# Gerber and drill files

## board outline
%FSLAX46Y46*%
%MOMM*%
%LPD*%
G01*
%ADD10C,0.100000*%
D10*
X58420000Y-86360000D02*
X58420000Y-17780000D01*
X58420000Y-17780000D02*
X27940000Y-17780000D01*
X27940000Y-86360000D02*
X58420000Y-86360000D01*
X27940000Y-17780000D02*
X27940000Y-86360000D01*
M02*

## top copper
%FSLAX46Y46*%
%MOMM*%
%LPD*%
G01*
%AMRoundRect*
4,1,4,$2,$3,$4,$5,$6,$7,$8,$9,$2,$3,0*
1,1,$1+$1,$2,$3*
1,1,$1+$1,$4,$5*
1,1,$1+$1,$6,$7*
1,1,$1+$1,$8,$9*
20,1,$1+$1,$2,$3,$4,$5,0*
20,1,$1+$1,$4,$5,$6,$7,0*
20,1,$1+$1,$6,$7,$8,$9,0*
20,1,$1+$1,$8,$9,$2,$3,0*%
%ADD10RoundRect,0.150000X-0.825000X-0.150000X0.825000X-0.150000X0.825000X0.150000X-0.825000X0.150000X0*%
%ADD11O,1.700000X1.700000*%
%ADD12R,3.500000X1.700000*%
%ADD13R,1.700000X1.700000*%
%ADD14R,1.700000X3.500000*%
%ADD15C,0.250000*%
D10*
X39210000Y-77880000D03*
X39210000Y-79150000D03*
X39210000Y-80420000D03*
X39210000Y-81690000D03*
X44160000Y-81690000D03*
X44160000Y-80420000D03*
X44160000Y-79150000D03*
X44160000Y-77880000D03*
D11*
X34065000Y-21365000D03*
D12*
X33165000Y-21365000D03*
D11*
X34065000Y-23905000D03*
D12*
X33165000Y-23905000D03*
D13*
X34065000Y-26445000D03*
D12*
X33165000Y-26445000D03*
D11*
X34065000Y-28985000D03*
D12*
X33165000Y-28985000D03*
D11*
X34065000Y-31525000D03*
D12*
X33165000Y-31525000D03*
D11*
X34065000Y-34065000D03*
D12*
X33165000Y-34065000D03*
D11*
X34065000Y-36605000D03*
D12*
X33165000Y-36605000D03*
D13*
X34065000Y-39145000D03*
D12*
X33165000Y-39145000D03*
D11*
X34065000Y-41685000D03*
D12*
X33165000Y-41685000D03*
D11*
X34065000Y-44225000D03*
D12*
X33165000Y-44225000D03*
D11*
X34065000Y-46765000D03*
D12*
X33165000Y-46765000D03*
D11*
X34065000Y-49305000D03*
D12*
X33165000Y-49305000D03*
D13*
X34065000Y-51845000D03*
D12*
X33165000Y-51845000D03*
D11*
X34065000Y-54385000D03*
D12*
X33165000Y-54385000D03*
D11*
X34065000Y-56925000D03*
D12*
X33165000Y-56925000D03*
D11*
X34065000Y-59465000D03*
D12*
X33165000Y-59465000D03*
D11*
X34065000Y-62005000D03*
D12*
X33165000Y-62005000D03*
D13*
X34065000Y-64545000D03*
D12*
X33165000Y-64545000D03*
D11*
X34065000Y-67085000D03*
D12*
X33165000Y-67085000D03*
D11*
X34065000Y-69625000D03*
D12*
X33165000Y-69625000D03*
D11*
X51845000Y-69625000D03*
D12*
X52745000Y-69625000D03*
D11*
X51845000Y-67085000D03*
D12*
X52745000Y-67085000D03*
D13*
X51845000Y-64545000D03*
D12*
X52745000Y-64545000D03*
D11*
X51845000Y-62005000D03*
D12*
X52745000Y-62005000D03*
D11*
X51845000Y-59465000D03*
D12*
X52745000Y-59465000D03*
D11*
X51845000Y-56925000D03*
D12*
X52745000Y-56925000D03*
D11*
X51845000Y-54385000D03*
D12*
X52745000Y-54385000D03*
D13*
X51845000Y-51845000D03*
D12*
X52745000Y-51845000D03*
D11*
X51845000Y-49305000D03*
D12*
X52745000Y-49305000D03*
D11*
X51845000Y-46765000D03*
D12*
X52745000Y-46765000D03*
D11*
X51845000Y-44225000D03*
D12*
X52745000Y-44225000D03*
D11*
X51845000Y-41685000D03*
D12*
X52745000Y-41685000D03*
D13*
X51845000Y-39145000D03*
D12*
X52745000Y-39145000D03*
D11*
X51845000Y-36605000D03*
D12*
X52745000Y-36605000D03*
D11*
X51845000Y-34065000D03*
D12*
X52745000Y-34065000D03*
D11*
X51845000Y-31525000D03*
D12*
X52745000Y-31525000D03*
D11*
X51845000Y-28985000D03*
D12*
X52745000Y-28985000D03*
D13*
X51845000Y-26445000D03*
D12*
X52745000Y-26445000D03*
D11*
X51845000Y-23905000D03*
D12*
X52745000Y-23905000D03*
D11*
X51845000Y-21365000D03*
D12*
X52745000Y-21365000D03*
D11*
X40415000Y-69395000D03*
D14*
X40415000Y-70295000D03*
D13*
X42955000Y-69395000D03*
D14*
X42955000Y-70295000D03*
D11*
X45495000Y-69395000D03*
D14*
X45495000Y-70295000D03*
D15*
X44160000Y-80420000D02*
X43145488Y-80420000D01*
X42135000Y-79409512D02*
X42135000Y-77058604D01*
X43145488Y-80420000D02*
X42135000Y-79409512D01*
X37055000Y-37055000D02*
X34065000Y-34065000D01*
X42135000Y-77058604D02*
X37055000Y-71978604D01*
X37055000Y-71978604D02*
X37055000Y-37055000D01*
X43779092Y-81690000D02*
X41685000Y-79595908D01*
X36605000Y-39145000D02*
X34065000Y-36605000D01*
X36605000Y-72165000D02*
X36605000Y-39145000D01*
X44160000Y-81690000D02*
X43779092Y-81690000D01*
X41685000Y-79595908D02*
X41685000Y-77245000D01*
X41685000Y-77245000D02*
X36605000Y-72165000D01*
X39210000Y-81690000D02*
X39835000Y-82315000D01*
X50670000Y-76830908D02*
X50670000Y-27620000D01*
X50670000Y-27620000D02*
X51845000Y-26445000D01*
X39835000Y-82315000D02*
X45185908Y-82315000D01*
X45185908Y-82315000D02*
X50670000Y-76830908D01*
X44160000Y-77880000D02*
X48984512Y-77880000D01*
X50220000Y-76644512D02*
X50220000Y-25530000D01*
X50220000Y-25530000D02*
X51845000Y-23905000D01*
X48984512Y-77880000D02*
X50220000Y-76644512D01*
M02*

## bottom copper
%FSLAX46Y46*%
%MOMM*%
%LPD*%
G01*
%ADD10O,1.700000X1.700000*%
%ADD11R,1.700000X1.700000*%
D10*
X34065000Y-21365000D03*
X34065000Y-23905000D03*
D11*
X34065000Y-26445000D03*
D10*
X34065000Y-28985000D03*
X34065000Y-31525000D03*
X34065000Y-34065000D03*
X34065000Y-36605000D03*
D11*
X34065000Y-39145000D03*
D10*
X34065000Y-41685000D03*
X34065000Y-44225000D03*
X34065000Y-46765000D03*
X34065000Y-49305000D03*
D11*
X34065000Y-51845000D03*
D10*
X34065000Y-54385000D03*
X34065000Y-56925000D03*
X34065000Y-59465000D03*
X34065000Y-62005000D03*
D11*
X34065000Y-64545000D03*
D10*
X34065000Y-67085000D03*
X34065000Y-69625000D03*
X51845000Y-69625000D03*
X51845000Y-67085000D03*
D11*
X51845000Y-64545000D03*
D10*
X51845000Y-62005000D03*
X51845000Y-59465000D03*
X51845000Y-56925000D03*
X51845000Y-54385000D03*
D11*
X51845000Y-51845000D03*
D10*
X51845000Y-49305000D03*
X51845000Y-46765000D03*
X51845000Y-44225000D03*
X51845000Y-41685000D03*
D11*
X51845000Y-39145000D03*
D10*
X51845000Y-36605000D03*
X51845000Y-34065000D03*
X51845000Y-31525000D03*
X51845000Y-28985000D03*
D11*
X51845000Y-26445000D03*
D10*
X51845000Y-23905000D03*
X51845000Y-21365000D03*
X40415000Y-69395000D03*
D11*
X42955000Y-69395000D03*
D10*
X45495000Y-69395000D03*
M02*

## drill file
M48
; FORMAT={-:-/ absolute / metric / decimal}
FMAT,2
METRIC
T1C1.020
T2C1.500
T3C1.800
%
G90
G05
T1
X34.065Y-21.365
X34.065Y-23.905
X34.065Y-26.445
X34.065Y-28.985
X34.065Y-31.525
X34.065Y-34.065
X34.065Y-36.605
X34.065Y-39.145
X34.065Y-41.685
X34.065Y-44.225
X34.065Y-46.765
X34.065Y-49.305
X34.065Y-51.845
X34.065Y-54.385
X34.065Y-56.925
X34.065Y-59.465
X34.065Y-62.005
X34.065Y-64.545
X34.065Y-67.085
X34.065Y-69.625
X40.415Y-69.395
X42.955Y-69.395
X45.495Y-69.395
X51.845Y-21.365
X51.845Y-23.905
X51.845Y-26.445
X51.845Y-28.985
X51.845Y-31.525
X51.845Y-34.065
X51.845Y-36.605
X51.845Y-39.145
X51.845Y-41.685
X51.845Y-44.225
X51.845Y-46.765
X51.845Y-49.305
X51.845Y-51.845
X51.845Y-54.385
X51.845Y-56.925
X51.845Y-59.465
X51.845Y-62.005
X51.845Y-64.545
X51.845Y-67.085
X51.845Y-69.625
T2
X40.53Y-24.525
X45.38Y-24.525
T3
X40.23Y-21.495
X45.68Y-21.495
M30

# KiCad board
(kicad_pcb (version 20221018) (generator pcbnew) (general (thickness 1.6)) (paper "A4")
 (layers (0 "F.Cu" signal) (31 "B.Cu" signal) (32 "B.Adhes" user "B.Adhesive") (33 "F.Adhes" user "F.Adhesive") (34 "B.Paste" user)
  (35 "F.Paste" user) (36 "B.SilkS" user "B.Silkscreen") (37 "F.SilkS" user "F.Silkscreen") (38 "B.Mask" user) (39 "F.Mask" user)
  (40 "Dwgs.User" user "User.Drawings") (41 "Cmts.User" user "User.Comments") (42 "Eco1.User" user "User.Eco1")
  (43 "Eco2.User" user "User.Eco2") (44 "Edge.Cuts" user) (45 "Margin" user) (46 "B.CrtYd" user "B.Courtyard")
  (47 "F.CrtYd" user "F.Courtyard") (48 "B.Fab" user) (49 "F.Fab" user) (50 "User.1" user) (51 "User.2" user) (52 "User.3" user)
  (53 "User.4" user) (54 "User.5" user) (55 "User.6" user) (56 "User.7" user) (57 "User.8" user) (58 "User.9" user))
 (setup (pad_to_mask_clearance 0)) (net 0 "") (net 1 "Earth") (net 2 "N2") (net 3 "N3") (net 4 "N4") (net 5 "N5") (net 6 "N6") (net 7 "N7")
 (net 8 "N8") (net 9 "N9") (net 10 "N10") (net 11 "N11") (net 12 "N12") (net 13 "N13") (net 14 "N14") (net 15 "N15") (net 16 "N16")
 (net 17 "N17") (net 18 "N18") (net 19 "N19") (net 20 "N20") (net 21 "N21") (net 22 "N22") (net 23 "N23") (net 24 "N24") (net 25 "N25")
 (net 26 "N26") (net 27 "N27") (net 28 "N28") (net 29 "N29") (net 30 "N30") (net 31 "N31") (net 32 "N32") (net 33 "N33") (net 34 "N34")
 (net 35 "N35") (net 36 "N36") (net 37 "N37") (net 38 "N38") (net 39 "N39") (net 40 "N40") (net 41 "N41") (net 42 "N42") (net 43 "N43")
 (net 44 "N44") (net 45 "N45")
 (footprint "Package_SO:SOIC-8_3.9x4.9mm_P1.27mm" (layer "F.Cu") (at 41.685 79.785)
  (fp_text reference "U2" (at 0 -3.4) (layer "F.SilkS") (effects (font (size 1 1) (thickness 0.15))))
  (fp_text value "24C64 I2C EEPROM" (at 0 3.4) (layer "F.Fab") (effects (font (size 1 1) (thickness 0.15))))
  (pad "1" smd roundrect (at -2.475 -1.905) (size 1.95 0.6) (layers "F.Cu" "F.Paste" "F.Mask") (roundrect_rratio 0.25) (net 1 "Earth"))
  (pad "2" smd roundrect (at -2.475 -0.635) (size 1.95 0.6) (layers "F.Cu" "F.Paste" "F.Mask") (roundrect_rratio 0.25) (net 1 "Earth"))
  (pad "3" smd roundrect (at -2.475 0.635) (size 1.95 0.6) (layers "F.Cu" "F.Paste" "F.Mask") (roundrect_rratio 0.25) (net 1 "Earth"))
  (pad "4" smd roundrect (at -2.475 1.905) (size 1.95 0.6) (layers "F.Cu" "F.Paste" "F.Mask") (roundrect_rratio 0.25) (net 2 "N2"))
  (pad "5" smd roundrect (at 2.475 1.905) (size 1.95 0.6) (layers "F.Cu" "F.Paste" "F.Mask") (roundrect_rratio 0.25) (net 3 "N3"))
  (pad "6" smd roundrect (at 2.475 0.635) (size 1.95 0.6) (layers "F.Cu" "F.Paste" "F.Mask") (roundrect_rratio 0.25) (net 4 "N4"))
  (pad "7" smd roundrect (at 2.475 -0.635) (size 1.95 0.6) (layers "F.Cu" "F.Paste" "F.Mask") (roundrect_rratio 0.25) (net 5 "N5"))
  (pad "8" smd roundrect (at 2.475 -1.905) (size 1.95 0.6) (layers "F.Cu" "F.Paste" "F.Mask") (roundrect_rratio 0.25) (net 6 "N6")))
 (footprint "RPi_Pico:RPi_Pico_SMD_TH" (layer "F.Cu") (at 42.955 45.495)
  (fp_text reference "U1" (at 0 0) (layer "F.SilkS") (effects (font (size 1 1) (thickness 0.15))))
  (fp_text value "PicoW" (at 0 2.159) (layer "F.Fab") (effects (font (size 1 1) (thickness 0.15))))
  (pad "" np_thru_hole oval (at -2.725 -24) (size 1.8 1.8) (drill 1.8) (layers "*.Cu" "*.Mask"))
  (pad "" np_thru_hole oval (at -2.425 -20.97) (size 1.5 1.5) (drill 1.5) (layers "*.Cu" "*.Mask"))
  (pad "" np_thru_hole oval (at 2.425 -20.97) (size 1.5 1.5) (drill 1.5) (layers "*.Cu" "*.Mask"))
  (pad "" np_thru_hole oval (at 2.725 -24) (size 1.8 1.8) (drill 1.8) (layers "*.Cu" "*.Mask"))
  (pad "1" thru_hole oval (at -8.89 -24.13) (size 1.7 1.7) (drill 1.02) (layers "*.Cu" "*.Mask") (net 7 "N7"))
  (pad "1" smd rect (at -8.89 -24.13) (size 3.5 1.7) (drill (offset -0.9 0)) (layers "F.Cu" "F.Mask") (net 7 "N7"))
  (pad "2" thru_hole oval (at -8.89 -21.59) (size 1.7 1.7) (drill 1.02) (layers "*.Cu" "*.Mask") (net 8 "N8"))
  (pad "2" smd rect (at -8.89 -21.59) (size 3.5 1.7) (drill (offset -0.9 0)) (layers "F.Cu" "F.Mask") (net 8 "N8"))
  (pad "3" thru_hole rect (at -8.89 -19.05) (size 1.7 1.7) (drill 1.02) (layers "*.Cu" "*.Mask") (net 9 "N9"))
  (pad "3" smd rect (at -8.89 -19.05) (size 3.5 1.7) (drill (offset -0.9 0)) (layers "F.Cu" "F.Mask") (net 9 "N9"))
  (pad "4" thru_hole oval (at -8.89 -16.51) (size 1.7 1.7) (drill 1.02) (layers "*.Cu" "*.Mask") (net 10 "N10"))
  (pad "4" smd rect (at -8.89 -16.51) (size 3.5 1.7) (drill (offset -0.9 0)) (layers "F.Cu" "F.Mask") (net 10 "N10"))
  (pad "5" thru_hole oval (at -8.89 -13.97) (size 1.7 1.7) (drill 1.02) (layers "*.Cu" "*.Mask") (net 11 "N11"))
  (pad "5" smd rect (at -8.89 -13.97) (size 3.5 1.7) (drill (offset -0.9 0)) (layers "F.Cu" "F.Mask") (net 11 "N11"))
  (pad "6" thru_hole oval (at -8.89 -11.43) (size 1.7 1.7) (drill 1.02) (layers "*.Cu" "*.Mask") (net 4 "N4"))
  (pad "6" smd rect (at -8.89 -11.43) (size 3.5 1.7) (drill (offset -0.9 0)) (layers "F.Cu" "F.Mask") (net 4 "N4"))
  (pad "7" thru_hole oval (at -8.89 -8.89) (size 1.7 1.7) (drill 1.02) (layers "*.Cu" "*.Mask") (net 3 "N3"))
  (pad "7" smd rect (at -8.89 -8.89) (size 3.5 1.7) (drill (offset -0.9 0)) (layers "F.Cu" "F.Mask") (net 3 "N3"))
  (pad "8" thru_hole rect (at -8.89 -6.35) (size 1.7 1.7) (drill 1.02) (layers "*.Cu" "*.Mask") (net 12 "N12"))
  (pad "8" smd rect (at -8.89 -6.35) (size 3.5 1.7) (drill (offset -0.9 0)) (layers "F.Cu" "F.Mask") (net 12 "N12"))
  (pad "9" thru_hole oval (at -8.89 -3.81) (size 1.7 1.7) (drill 1.02) (layers "*.Cu" "*.Mask") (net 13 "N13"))
  (pad "9" smd rect (at -8.89 -3.81) (size 3.5 1.7) (drill (offset -0.9 0)) (layers "F.Cu" "F.Mask") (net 13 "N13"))
  (pad "10" thru_hole oval (at -8.89 -1.27) (size 1.7 1.7) (drill 1.02) (layers "*.Cu" "*.Mask") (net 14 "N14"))
  (pad "10" smd rect (at -8.89 -1.27) (size 3.5 1.7) (drill (offset -0.9 0)) (layers "F.Cu" "F.Mask") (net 14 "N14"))
  (pad "11" thru_hole oval (at -8.89 1.27) (size 1.7 1.7) (drill 1.02) (layers "*.Cu" "*.Mask") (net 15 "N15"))
  (pad "11" smd rect (at -8.89 1.27) (size 3.5 1.7) (drill (offset -0.9 0)) (layers "F.Cu" "F.Mask") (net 15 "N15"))
  (pad "12" thru_hole oval (at -8.89 3.81) (size 1.7 1.7) (drill 1.02) (layers "*.Cu" "*.Mask") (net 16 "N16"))
  (pad "12" smd rect (at -8.89 3.81) (size 3.5 1.7) (drill (offset -0.9 0)) (layers "F.Cu" "F.Mask") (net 16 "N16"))
  (pad "13" thru_hole rect (at -8.89 6.35) (size 1.7 1.7) (drill 1.02) (layers "*.Cu" "*.Mask") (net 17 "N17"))
  (pad "13" smd rect (at -8.89 6.35) (size 3.5 1.7) (drill (offset -0.9 0)) (layers "F.Cu" "F.Mask") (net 17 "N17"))
  (pad "14" thru_hole oval (at -8.89 8.89) (size 1.7 1.7) (drill 1.02) (layers "*.Cu" "*.Mask") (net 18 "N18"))
  (pad "14" smd rect (at -8.89 8.89) (size 3.5 1.7) (drill (offset -0.9 0)) (layers "F.Cu" "F.Mask") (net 18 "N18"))
  (pad "15" thru_hole oval (at -8.89 11.43) (size 1.7 1.7) (drill 1.02) (layers "*.Cu" "*.Mask") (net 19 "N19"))
  (pad "15" smd rect (at -8.89 11.43) (size 3.5 1.7) (drill (offset -0.9 0)) (layers "F.Cu" "F.Mask") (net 19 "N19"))
  (pad "16" thru_hole oval (at -8.89 13.97) (size 1.7 1.7) (drill 1.02) (layers "*.Cu" "*.Mask") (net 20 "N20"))
  (pad "16" smd rect (at -8.89 13.97) (size 3.5 1.7) (drill (offset -0.9 0)) (layers "F.Cu" "F.Mask") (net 20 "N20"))
  (pad "17" thru_hole oval (at -8.89 16.51) (size 1.7 1.7) (drill 1.02) (layers "*.Cu" "*.Mask") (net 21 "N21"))
  (pad "17" smd rect (at -8.89 16.51) (size 3.5 1.7) (drill (offset -0.9 0)) (layers "F.Cu" "F.Mask") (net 21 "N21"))
  (pad "18" thru_hole rect (at -8.89 19.05) (size 1.7 1.7) (drill 1.02) (layers "*.Cu" "*.Mask") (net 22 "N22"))
  (pad "18" smd rect (at -8.89 19.05) (size 3.5 1.7) (drill (offset -0.9 0)) (layers "F.Cu" "F.Mask") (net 22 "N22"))
  (pad "19" thru_hole oval (at -8.89 21.59) (size 1.7 1.7) (drill 1.02) (layers "*.Cu" "*.Mask") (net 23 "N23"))
  (pad "19" smd rect (at -8.89 21.59) (size 3.5 1.7) (drill (offset -0.9 0)) (layers "F.Cu" "F.Mask") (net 23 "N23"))
  (pad "20" thru_hole oval (at -8.89 24.13) (size 1.7 1.7) (drill 1.02) (layers "*.Cu" "*.Mask") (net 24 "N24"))
  (pad "20" smd rect (at -8.89 24.13) (size 3.5 1.7) (drill (offset -0.9 0)) (layers "F.Cu" "F.Mask") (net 24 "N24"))
  (pad "21" thru_hole oval (at 8.89 24.13) (size 1.7 1.7) (drill 1.02) (layers "*.Cu" "*.Mask") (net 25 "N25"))
  (pad "21" smd rect (at 8.89 24.13) (size 3.5 1.7) (drill (offset 0.9 0)) (layers "F.Cu" "F.Mask") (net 25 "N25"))
  (pad "22" thru_hole oval (at 8.89 21.59) (size 1.7 1.7) (drill 1.02) (layers "*.Cu" "*.Mask") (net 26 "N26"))
  (pad "22" smd rect (at 8.89 21.59) (size 3.5 1.7) (drill (offset 0.9 0)) (layers "F.Cu" "F.Mask") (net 26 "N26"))
  (pad "23" thru_hole rect (at 8.89 19.05) (size 1.7 1.7) (drill 1.02) (layers "*.Cu" "*.Mask") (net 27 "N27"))
  (pad "23" smd rect (at 8.89 19.05) (size 3.5 1.7) (drill (offset 0.9 0)) (layers "F.Cu" "F.Mask") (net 27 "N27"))
  (pad "24" thru_hole oval (at 8.89 16.51) (size 1.7 1.7) (drill 1.02) (layers "*.Cu" "*.Mask") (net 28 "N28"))
  (pad "24" smd rect (at 8.89 16.51) (size 3.5 1.7) (drill (offset 0.9 0)) (layers "F.Cu" "F.Mask") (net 28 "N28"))
  (pad "25" thru_hole oval (at 8.89 13.97) (size 1.7 1.7) (drill 1.02) (layers "*.Cu" "*.Mask") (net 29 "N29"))
  (pad "25" smd rect (at 8.89 13.97) (size 3.5 1.7) (drill (offset 0.9 0)) (layers "F.Cu" "F.Mask") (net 29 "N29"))
  (pad "26" thru_hole oval (at 8.89 11.43) (size 1.7 1.7) (drill 1.02) (layers "*.Cu" "*.Mask") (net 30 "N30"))
  (pad "26" smd rect (at 8.89 11.43) (size 3.5 1.7) (drill (offset 0.9 0)) (layers "F.Cu" "F.Mask") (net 30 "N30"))
  (pad "27" thru_hole oval (at 8.89 8.89) (size 1.7 1.7) (drill 1.02) (layers "*.Cu" "*.Mask") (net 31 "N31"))
  (pad "27" smd rect (at 8.89 8.89) (size 3.5 1.7) (drill (offset 0.9 0)) (layers "F.Cu" "F.Mask") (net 31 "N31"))
  (pad "28" thru_hole rect (at 8.89 6.35) (size 1.7 1.7) (drill 1.02) (layers "*.Cu" "*.Mask") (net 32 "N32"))
  (pad "28" smd rect (at 8.89 6.35) (size 3.5 1.7) (drill (offset 0.9 0)) (layers "F.Cu" "F.Mask") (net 32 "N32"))
  (pad "29" thru_hole oval (at 8.89 3.81) (size 1.7 1.7) (drill 1.02) (layers "*.Cu" "*.Mask") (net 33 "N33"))
  (pad "29" smd rect (at 8.89 3.81) (size 3.5 1.7) (drill (offset 0.9 0)) (layers "F.Cu" "F.Mask") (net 33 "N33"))
  (pad "30" thru_hole oval (at 8.89 1.27) (size 1.7 1.7) (drill 1.02) (layers "*.Cu" "*.Mask") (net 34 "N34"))
  (pad "30" smd rect (at 8.89 1.27) (size 3.5 1.7) (drill (offset 0.9 0)) (layers "F.Cu" "F.Mask") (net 34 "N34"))
  (pad "31" thru_hole oval (at 8.89 -1.27) (size 1.7 1.7) (drill 1.02) (layers "*.Cu" "*.Mask") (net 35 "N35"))
  (pad "31" smd rect (at 8.89 -1.27) (size 3.5 1.7) (drill (offset 0.9 0)) (layers "F.Cu" "F.Mask") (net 35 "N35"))
  (pad "32" thru_hole oval (at 8.89 -3.81) (size 1.7 1.7) (drill 1.02) (layers "*.Cu" "*.Mask") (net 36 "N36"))
  (pad "32" smd rect (at 8.89 -3.81) (size 3.5 1.7) (drill (offset 0.9 0)) (layers "F.Cu" "F.Mask") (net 36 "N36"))
  (pad "33" thru_hole rect (at 8.89 -6.35) (size 1.7 1.7) (drill 1.02) (layers "*.Cu" "*.Mask") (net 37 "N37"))
  (pad "33" smd rect (at 8.89 -6.35) (size 3.5 1.7) (drill (offset 0.9 0)) (layers "F.Cu" "F.Mask") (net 37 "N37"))
  (pad "34" thru_hole oval (at 8.89 -8.89) (size 1.7 1.7) (drill 1.02) (layers "*.Cu" "*.Mask") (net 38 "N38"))
  (pad "34" smd rect (at 8.89 -8.89) (size 3.5 1.7) (drill (offset 0.9 0)) (layers "F.Cu" "F.Mask") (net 38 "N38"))
  (pad "35" thru_hole oval (at 8.89 -11.43) (size 1.7 1.7) (drill 1.02) (layers "*.Cu" "*.Mask") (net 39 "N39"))
  (pad "35" smd rect (at 8.89 -11.43) (size 3.5 1.7) (drill (offset 0.9 0)) (layers "F.Cu" "F.Mask") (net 39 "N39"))
  (pad "36" thru_hole oval (at 8.89 -13.97) (size 1.7 1.7) (drill 1.02) (layers "*.Cu" "*.Mask") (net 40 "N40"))
  (pad "36" smd rect (at 8.89 -13.97) (size 3.5 1.7) (drill (offset 0.9 0)) (layers "F.Cu" "F.Mask") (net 40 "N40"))
  (pad "37" thru_hole oval (at 8.89 -16.51) (size 1.7 1.7) (drill 1.02) (layers "*.Cu" "*.Mask") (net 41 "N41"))
  (pad "37" smd rect (at 8.89 -16.51) (size 3.5 1.7) (drill (offset 0.9 0)) (layers "F.Cu" "F.Mask") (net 41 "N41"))
  (pad "38" thru_hole rect (at 8.89 -19.05) (size 1.7 1.7) (drill 1.02) (layers "*.Cu" "*.Mask") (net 2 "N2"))
  (pad "38" smd rect (at 8.89 -19.05) (size 3.5 1.7) (drill (offset 0.9 0)) (layers "F.Cu" "F.Mask") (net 2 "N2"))
  (pad "39" thru_hole oval (at 8.89 -21.59) (size 1.7 1.7) (drill 1.02) (layers "*.Cu" "*.Mask") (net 6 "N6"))
  (pad "39" smd rect (at 8.89 -21.59) (size 3.5 1.7) (drill (offset 0.9 0)) (layers "F.Cu" "F.Mask") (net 6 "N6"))
  (pad "40" thru_hole oval (at 8.89 -24.13) (size 1.7 1.7) (drill 1.02) (layers "*.Cu" "*.Mask") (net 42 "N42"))
  (pad "40" smd rect (at 8.89 -24.13) (size 3.5 1.7) (drill (offset 0.9 0)) (layers "F.Cu" "F.Mask") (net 42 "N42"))
  (pad "41" thru_hole oval (at -2.54 23.9) (size 1.7 1.7) (drill 1.02) (layers "*.Cu" "*.Mask") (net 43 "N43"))
  (pad "41" smd rect (at -2.54 23.9 90) (size 3.5 1.7) (drill (offset -0.9 0)) (layers "F.Cu" "F.Mask") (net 43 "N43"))
  (pad "42" thru_hole rect (at 0 23.9) (size 1.7 1.7) (drill 1.02) (layers "*.Cu" "*.Mask") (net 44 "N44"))
  (pad "42" smd rect (at 0 23.9 90) (size 3.5 1.7) (drill (offset -0.9 0)) (layers "F.Cu" "F.Mask") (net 44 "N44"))
  (pad "43" thru_hole oval (at 2.54 23.9) (size 1.7 1.7) (drill 1.02) (layers "*.Cu" "*.Mask") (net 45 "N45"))
  (pad "43" smd rect (at 2.54 23.9 90) (size 3.5 1.7) (drill (offset -0.9 0)) (layers "F.Cu" "F.Mask") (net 45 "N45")))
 (gr_line (start 58.42 86.36) (end 58.42 17.78) (stroke (width 0.1) (type default)) (layer "Edge.Cuts"))
 (gr_line (start 58.42 17.78) (end 27.94 17.78) (stroke (width 0.1) (type default)) (layer "Edge.Cuts"))
 (gr_line (start 27.94 86.36) (end 58.42 86.36) (stroke (width 0.1) (type default)) (layer "Edge.Cuts"))
 (gr_line (start 27.94 17.78) (end 27.94 86.36) (stroke (width 0.1) (type default)) (layer "Edge.Cuts"))
 (segment (start 44.16 80.42) (end 43.145488 80.42) (width 0.25) (layer "F.Cu") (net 4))
 (segment (start 42.135 79.409512) (end 42.135 77.058604) (width 0.25) (layer "F.Cu") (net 4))
 (segment (start 43.145488 80.42) (end 42.135 79.409512) (width 0.25) (layer "F.Cu") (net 4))
 (segment (start 37.055 37.055) (end 34.065 34.065) (width 0.25) (layer "F.Cu") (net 4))
 (segment (start 42.135 77.058604) (end 37.055 71.978604) (width 0.25) (layer "F.Cu") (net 4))
 (segment (start 37.055 71.978604) (end 37.055 37.055) (width 0.25) (layer "F.Cu") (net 4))
 (segment (start 43.779092 81.69) (end 41.685 79.595908) (width 0.25) (layer "F.Cu") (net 3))
 (segment (start 36.605 39.145) (end 34.065 36.605) (width 0.25) (layer "F.Cu") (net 3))
 (segment (start 36.605 72.165) (end 36.605 39.145) (width 0.25) (layer "F.Cu") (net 3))
 (segment (start 44.16 81.69) (end 43.779092 81.69) (width 0.25) (layer "F.Cu") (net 3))
 (segment (start 41.685 79.595908) (end 41.685 77.245) (width 0.25) (layer "F.Cu") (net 3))
 (segment (start 41.685 77.245) (end 36.605 72.165) (width 0.25) (layer "F.Cu") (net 3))
 (segment (start 39.21 81.69) (end 39.835 82.315) (width 0.25) (layer "F.Cu") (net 2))
 (segment (start 50.67 76.830908) (end 50.67 27.62) (width 0.25) (layer "F.Cu") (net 2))
 (segment (start 50.67 27.62) (end 51.845 26.445) (width 0.25) (layer "F.Cu") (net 2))
 (segment (start 39.835 82.315) (end 45.185908 82.315) (width 0.25) (layer "F.Cu") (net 2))
 (segment (start 45.185908 82.315) (end 50.67 76.830908) (width 0.25) (layer "F.Cu") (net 2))
 (segment (start 44.16 77.88) (end 48.984512 77.88) (width 0.25) (layer "F.Cu") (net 6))
 (segment (start 50.22 76.644512) (end 50.22 25.53) (width 0.25) (layer "F.Cu") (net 6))
 (segment (start 50.22 25.53) (end 51.845 23.905) (width 0.25) (layer "F.Cu") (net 6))
 (segment (start 48.984512 77.88) (end 50.22 76.644512) (width 0.25) (layer "F.Cu") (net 6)))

